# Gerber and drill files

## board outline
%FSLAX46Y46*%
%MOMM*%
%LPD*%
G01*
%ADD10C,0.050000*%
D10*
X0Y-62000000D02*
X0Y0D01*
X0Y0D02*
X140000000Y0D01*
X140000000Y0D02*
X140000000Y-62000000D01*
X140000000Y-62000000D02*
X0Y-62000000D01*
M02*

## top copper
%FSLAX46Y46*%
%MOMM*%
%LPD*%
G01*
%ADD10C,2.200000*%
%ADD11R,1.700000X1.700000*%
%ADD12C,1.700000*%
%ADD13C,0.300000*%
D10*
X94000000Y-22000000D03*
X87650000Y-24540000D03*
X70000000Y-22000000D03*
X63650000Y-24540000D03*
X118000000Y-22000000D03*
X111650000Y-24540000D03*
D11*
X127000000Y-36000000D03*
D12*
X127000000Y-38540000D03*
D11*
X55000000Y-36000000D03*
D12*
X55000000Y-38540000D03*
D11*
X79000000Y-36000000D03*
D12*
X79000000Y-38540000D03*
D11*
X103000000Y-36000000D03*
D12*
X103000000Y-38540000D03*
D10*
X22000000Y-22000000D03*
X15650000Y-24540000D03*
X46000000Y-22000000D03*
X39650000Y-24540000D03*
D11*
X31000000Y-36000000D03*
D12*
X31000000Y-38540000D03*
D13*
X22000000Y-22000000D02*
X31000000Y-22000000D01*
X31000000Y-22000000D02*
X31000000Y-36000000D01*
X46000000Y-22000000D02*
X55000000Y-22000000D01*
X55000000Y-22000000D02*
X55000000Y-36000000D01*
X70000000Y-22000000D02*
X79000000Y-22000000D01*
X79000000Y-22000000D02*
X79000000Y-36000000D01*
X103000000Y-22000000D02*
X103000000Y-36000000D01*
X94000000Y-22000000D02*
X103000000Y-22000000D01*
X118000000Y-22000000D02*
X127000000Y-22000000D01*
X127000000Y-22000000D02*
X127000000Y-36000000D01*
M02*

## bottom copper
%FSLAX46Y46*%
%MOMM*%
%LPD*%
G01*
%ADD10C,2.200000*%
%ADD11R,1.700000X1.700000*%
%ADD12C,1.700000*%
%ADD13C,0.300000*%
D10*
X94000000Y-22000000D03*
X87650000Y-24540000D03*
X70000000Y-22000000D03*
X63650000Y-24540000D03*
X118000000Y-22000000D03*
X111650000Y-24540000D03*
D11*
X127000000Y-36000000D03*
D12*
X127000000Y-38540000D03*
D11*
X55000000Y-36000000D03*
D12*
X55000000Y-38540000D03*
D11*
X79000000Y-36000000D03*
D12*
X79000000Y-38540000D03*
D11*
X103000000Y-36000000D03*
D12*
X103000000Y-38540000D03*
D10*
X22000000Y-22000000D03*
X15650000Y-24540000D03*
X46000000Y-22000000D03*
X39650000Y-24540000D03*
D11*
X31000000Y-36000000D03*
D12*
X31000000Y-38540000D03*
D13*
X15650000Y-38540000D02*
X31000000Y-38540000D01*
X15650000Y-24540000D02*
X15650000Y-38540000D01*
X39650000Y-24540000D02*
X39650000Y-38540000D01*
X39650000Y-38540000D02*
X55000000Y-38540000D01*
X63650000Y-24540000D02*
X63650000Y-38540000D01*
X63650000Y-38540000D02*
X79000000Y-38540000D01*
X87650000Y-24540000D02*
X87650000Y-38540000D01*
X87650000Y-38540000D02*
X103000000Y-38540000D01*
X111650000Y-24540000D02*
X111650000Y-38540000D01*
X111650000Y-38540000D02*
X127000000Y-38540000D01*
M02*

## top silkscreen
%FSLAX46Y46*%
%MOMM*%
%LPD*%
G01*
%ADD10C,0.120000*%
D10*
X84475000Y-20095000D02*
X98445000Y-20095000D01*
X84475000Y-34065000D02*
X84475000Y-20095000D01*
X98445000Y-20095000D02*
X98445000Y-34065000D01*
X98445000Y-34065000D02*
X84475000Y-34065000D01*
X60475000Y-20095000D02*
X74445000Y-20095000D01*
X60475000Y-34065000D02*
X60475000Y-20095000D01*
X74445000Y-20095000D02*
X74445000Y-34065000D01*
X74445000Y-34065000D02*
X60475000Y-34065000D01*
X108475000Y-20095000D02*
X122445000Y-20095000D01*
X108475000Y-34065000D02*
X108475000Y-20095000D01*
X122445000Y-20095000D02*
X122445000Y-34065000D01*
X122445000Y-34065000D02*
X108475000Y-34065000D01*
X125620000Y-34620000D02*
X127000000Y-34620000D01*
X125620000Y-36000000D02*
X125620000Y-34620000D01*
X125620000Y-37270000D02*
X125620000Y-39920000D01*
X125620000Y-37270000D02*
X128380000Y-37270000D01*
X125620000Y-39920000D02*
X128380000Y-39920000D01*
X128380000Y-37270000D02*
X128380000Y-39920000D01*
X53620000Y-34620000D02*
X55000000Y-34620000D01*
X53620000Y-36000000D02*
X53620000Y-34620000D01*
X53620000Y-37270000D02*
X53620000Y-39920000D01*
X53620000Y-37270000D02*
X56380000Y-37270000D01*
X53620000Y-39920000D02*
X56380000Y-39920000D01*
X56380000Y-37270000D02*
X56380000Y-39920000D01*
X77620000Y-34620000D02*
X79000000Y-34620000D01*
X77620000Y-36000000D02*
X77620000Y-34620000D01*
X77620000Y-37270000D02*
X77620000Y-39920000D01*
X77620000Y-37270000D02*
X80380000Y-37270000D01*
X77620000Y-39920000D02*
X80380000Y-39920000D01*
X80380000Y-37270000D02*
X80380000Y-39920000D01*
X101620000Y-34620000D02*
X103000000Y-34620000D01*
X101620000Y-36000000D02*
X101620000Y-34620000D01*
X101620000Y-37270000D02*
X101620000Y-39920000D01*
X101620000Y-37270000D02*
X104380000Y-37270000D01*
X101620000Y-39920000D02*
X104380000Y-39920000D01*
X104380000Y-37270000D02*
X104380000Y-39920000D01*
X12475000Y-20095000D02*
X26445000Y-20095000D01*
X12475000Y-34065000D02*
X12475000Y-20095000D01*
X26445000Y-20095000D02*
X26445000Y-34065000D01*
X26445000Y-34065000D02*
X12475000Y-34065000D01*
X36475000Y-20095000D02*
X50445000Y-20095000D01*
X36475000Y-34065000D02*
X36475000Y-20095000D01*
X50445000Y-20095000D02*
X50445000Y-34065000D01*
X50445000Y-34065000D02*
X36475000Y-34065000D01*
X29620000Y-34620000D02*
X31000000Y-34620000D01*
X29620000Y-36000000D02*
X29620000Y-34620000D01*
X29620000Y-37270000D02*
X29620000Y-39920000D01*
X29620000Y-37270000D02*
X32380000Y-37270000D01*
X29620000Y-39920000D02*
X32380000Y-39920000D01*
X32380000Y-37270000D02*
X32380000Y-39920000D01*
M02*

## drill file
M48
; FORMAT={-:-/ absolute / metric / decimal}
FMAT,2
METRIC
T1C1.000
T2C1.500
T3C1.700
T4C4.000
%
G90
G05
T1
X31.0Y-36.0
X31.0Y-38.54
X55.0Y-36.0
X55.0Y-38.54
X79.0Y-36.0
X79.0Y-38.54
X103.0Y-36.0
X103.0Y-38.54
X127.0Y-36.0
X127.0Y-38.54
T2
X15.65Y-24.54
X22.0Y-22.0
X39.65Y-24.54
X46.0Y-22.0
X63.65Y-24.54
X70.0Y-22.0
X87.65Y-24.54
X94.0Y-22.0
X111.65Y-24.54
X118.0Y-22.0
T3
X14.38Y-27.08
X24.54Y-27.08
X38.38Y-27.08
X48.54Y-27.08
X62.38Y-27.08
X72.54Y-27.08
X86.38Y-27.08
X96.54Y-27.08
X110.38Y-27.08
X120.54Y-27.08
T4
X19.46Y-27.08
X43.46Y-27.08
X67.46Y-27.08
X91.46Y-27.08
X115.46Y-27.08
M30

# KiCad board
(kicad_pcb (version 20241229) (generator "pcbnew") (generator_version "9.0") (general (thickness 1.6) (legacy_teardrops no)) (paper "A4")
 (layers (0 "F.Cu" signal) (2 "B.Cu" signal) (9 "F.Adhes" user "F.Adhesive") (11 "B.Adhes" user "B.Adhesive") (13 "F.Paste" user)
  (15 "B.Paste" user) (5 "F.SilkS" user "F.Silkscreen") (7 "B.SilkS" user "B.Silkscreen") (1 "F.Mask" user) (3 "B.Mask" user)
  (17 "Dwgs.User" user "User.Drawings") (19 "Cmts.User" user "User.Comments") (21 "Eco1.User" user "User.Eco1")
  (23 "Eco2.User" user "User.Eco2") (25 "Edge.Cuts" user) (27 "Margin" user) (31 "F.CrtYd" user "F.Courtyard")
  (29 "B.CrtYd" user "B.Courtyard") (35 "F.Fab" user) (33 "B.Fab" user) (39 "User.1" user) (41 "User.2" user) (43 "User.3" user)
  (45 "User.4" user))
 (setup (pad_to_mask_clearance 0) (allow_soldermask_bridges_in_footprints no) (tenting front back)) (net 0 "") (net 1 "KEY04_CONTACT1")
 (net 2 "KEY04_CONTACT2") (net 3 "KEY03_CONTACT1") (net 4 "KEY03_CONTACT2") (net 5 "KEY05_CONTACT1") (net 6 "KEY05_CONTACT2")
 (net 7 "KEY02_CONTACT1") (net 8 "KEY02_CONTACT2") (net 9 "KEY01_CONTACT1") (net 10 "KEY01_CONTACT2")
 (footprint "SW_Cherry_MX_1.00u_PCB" (layer "F.Cu") (at 94 22)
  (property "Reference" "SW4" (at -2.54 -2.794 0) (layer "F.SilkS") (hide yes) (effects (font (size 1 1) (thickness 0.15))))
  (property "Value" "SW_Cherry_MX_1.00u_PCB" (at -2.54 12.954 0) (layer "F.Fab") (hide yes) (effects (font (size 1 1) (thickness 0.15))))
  (fp_line (start -9.525 -1.905) (end 4.445 -1.905) (stroke (width 0.12) (type solid)) (layer "F.SilkS"))
  (fp_line (start -9.525 12.065) (end -9.525 -1.905) (stroke (width 0.12) (type solid)) (layer "F.SilkS"))
  (fp_line (start 4.445 -1.905) (end 4.445 12.065) (stroke (width 0.12) (type solid)) (layer "F.SilkS"))
  (fp_line (start 4.445 12.065) (end -9.525 12.065) (stroke (width 0.12) (type solid)) (layer "F.SilkS"))
  (pad "" np_thru_hole circle (at -7.62 5.08) (size 1.7 1.7) (drill 1.7) (layers "*.Cu" "*.Mask"))
  (pad "" np_thru_hole circle (at -2.54 5.08) (size 4 4) (drill 4) (layers "*.Cu" "*.Mask"))
  (pad "" np_thru_hole circle (at 2.54 5.08) (size 1.7 1.7) (drill 1.7) (layers "*.Cu" "*.Mask"))
  (pad "1" thru_hole circle (at 0 0) (size 2.2 2.2) (drill 1.5) (layers "*.Cu" "*.Mask") (remove_unused_layers no) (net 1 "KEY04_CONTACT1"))
  (pad "2" thru_hole circle (at -6.35 2.54) (size 2.2 2.2) (drill 1.5) (layers "*.Cu" "*.Mask") (remove_unused_layers no)
   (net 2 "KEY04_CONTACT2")))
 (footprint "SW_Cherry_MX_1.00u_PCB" (layer "F.Cu") (at 70 22)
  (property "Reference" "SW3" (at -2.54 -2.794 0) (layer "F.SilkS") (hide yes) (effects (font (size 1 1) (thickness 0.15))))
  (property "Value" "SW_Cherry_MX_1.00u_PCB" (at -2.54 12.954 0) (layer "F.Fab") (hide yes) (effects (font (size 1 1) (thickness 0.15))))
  (fp_line (start -9.525 -1.905) (end 4.445 -1.905) (stroke (width 0.12) (type solid)) (layer "F.SilkS"))
  (fp_line (start -9.525 12.065) (end -9.525 -1.905) (stroke (width 0.12) (type solid)) (layer "F.SilkS"))
  (fp_line (start 4.445 -1.905) (end 4.445 12.065) (stroke (width 0.12) (type solid)) (layer "F.SilkS"))
  (fp_line (start 4.445 12.065) (end -9.525 12.065) (stroke (width 0.12) (type solid)) (layer "F.SilkS"))
  (pad "" np_thru_hole circle (at -7.62 5.08) (size 1.7 1.7) (drill 1.7) (layers "*.Cu" "*.Mask"))
  (pad "" np_thru_hole circle (at -2.54 5.08) (size 4 4) (drill 4) (layers "*.Cu" "*.Mask"))
  (pad "" np_thru_hole circle (at 2.54 5.08) (size 1.7 1.7) (drill 1.7) (layers "*.Cu" "*.Mask"))
  (pad "1" thru_hole circle (at 0 0) (size 2.2 2.2) (drill 1.5) (layers "*.Cu" "*.Mask") (remove_unused_layers no) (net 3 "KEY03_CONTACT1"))
  (pad "2" thru_hole circle (at -6.35 2.54) (size 2.2 2.2) (drill 1.5) (layers "*.Cu" "*.Mask") (remove_unused_layers no)
   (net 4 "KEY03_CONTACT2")))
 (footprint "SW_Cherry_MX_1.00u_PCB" (layer "F.Cu") (at 118 22)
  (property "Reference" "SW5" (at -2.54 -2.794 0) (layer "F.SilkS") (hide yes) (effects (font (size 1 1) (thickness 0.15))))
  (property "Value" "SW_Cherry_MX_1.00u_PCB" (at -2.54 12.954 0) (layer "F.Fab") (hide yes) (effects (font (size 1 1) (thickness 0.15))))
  (fp_line (start -9.525 -1.905) (end 4.445 -1.905) (stroke (width 0.12) (type solid)) (layer "F.SilkS"))
  (fp_line (start -9.525 12.065) (end -9.525 -1.905) (stroke (width 0.12) (type solid)) (layer "F.SilkS"))
  (fp_line (start 4.445 -1.905) (end 4.445 12.065) (stroke (width 0.12) (type solid)) (layer "F.SilkS"))
  (fp_line (start 4.445 12.065) (end -9.525 12.065) (stroke (width 0.12) (type solid)) (layer "F.SilkS"))
  (pad "" np_thru_hole circle (at -7.62 5.08) (size 1.7 1.7) (drill 1.7) (layers "*.Cu" "*.Mask"))
  (pad "" np_thru_hole circle (at -2.54 5.08) (size 4 4) (drill 4) (layers "*.Cu" "*.Mask"))
  (pad "" np_thru_hole circle (at 2.54 5.08) (size 1.7 1.7) (drill 1.7) (layers "*.Cu" "*.Mask"))
  (pad "1" thru_hole circle (at 0 0) (size 2.2 2.2) (drill 1.5) (layers "*.Cu" "*.Mask") (remove_unused_layers no) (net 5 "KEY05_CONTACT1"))
  (pad "2" thru_hole circle (at -6.35 2.54) (size 2.2 2.2) (drill 1.5) (layers "*.Cu" "*.Mask") (remove_unused_layers no)
   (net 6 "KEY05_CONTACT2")))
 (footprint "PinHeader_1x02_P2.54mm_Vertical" (layer "F.Cu") (at 127 36)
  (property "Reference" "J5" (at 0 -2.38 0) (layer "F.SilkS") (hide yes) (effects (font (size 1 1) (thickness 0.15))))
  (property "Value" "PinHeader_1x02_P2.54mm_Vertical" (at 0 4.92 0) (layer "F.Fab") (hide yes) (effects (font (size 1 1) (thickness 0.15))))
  (fp_line (start -1.38 -1.38) (end 0 -1.38) (stroke (width 0.12) (type solid)) (layer "F.SilkS"))
  (fp_line (start -1.38 0) (end -1.38 -1.38) (stroke (width 0.12) (type solid)) (layer "F.SilkS"))
  (fp_line (start -1.38 1.27) (end -1.38 3.92) (stroke (width 0.12) (type solid)) (layer "F.SilkS"))
  (fp_line (start -1.38 1.27) (end 1.38 1.27) (stroke (width 0.12) (type solid)) (layer "F.SilkS"))
  (fp_line (start -1.38 3.92) (end 1.38 3.92) (stroke (width 0.12) (type solid)) (layer "F.SilkS"))
  (fp_line (start 1.38 1.27) (end 1.38 3.92) (stroke (width 0.12) (type solid)) (layer "F.SilkS"))
  (pad "1" thru_hole rect (at 0 0) (size 1.7 1.7) (drill 1) (layers "*.Cu" "*.Mask") (remove_unused_layers no) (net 5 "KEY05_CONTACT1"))
  (pad "2" thru_hole circle (at 0 2.54) (size 1.7 1.7) (drill 1) (layers "*.Cu" "*.Mask") (remove_unused_layers no) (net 6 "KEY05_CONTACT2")))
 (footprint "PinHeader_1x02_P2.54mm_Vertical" (layer "F.Cu") (at 55 36)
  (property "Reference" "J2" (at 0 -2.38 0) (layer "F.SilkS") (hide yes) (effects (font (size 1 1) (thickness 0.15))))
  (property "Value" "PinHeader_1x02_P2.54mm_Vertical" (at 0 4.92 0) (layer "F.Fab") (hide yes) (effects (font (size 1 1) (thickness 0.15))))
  (fp_line (start -1.38 -1.38) (end 0 -1.38) (stroke (width 0.12) (type solid)) (layer "F.SilkS"))
  (fp_line (start -1.38 0) (end -1.38 -1.38) (stroke (width 0.12) (type solid)) (layer "F.SilkS"))
  (fp_line (start -1.38 1.27) (end -1.38 3.92) (stroke (width 0.12) (type solid)) (layer "F.SilkS"))
  (fp_line (start -1.38 1.27) (end 1.38 1.27) (stroke (width 0.12) (type solid)) (layer "F.SilkS"))
  (fp_line (start -1.38 3.92) (end 1.38 3.92) (stroke (width 0.12) (type solid)) (layer "F.SilkS"))
  (fp_line (start 1.38 1.27) (end 1.38 3.92) (stroke (width 0.12) (type solid)) (layer "F.SilkS"))
  (pad "1" thru_hole rect (at 0 0) (size 1.7 1.7) (drill 1) (layers "*.Cu" "*.Mask") (remove_unused_layers no) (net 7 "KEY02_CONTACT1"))
  (pad "2" thru_hole circle (at 0 2.54) (size 1.7 1.7) (drill 1) (layers "*.Cu" "*.Mask") (remove_unused_layers no) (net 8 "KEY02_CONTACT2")))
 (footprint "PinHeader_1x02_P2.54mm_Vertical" (layer "F.Cu") (at 79 36)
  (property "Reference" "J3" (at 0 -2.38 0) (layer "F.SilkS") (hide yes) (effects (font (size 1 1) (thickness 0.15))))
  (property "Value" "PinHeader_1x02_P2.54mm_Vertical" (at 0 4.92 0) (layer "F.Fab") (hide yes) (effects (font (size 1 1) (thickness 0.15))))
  (fp_line (start -1.38 -1.38) (end 0 -1.38) (stroke (width 0.12) (type solid)) (layer "F.SilkS"))
  (fp_line (start -1.38 0) (end -1.38 -1.38) (stroke (width 0.12) (type solid)) (layer "F.SilkS"))
  (fp_line (start -1.38 1.27) (end -1.38 3.92) (stroke (width 0.12) (type solid)) (layer "F.SilkS"))
  (fp_line (start -1.38 1.27) (end 1.38 1.27) (stroke (width 0.12) (type solid)) (layer "F.SilkS"))
  (fp_line (start -1.38 3.92) (end 1.38 3.92) (stroke (width 0.12) (type solid)) (layer "F.SilkS"))
  (fp_line (start 1.38 1.27) (end 1.38 3.92) (stroke (width 0.12) (type solid)) (layer "F.SilkS"))
  (pad "1" thru_hole rect (at 0 0) (size 1.7 1.7) (drill 1) (layers "*.Cu" "*.Mask") (remove_unused_layers no) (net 3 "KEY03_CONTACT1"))
  (pad "2" thru_hole circle (at 0 2.54) (size 1.7 1.7) (drill 1) (layers "*.Cu" "*.Mask") (remove_unused_layers no) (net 4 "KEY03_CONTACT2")))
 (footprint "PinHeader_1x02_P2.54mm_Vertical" (layer "F.Cu") (at 103 36)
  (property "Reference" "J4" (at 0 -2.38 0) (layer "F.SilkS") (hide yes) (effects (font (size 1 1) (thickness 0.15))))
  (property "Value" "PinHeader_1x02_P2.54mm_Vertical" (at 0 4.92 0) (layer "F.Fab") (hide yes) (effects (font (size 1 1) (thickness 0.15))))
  (fp_line (start -1.38 -1.38) (end 0 -1.38) (stroke (width 0.12) (type solid)) (layer "F.SilkS"))
  (fp_line (start -1.38 0) (end -1.38 -1.38) (stroke (width 0.12) (type solid)) (layer "F.SilkS"))
  (fp_line (start -1.38 1.27) (end -1.38 3.92) (stroke (width 0.12) (type solid)) (layer "F.SilkS"))
  (fp_line (start -1.38 1.27) (end 1.38 1.27) (stroke (width 0.12) (type solid)) (layer "F.SilkS"))
  (fp_line (start -1.38 3.92) (end 1.38 3.92) (stroke (width 0.12) (type solid)) (layer "F.SilkS"))
  (fp_line (start 1.38 1.27) (end 1.38 3.92) (stroke (width 0.12) (type solid)) (layer "F.SilkS"))
  (pad "1" thru_hole rect (at 0 0) (size 1.7 1.7) (drill 1) (layers "*.Cu" "*.Mask") (remove_unused_layers no) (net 1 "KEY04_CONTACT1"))
  (pad "2" thru_hole circle (at 0 2.54) (size 1.7 1.7) (drill 1) (layers "*.Cu" "*.Mask") (remove_unused_layers no) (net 2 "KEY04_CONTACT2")))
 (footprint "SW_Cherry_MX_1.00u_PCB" (layer "F.Cu") (at 22 22)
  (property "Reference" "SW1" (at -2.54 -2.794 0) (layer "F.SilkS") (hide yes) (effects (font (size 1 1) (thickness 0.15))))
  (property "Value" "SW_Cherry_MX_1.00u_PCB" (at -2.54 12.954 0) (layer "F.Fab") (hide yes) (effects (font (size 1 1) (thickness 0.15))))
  (fp_line (start -9.525 -1.905) (end 4.445 -1.905) (stroke (width 0.12) (type solid)) (layer "F.SilkS"))
  (fp_line (start -9.525 12.065) (end -9.525 -1.905) (stroke (width 0.12) (type solid)) (layer "F.SilkS"))
  (fp_line (start 4.445 -1.905) (end 4.445 12.065) (stroke (width 0.12) (type solid)) (layer "F.SilkS"))
  (fp_line (start 4.445 12.065) (end -9.525 12.065) (stroke (width 0.12) (type solid)) (layer "F.SilkS"))
  (pad "" np_thru_hole circle (at -7.62 5.08) (size 1.7 1.7) (drill 1.7) (layers "*.Cu" "*.Mask"))
  (pad "" np_thru_hole circle (at -2.54 5.08) (size 4 4) (drill 4) (layers "*.Cu" "*.Mask"))
  (pad "" np_thru_hole circle (at 2.54 5.08) (size 1.7 1.7) (drill 1.7) (layers "*.Cu" "*.Mask"))
  (pad "1" thru_hole circle (at 0 0) (size 2.2 2.2) (drill 1.5) (layers "*.Cu" "*.Mask") (remove_unused_layers no) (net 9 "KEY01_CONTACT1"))
  (pad "2" thru_hole circle (at -6.35 2.54) (size 2.2 2.2) (drill 1.5) (layers "*.Cu" "*.Mask") (remove_unused_layers no)
   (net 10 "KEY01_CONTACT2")))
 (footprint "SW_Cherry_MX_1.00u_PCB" (layer "F.Cu") (at 46 22)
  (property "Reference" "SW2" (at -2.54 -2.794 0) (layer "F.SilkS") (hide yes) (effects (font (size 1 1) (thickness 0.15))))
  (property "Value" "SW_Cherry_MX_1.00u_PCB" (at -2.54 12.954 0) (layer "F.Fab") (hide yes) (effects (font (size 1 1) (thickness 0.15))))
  (fp_line (start -9.525 -1.905) (end 4.445 -1.905) (stroke (width 0.12) (type solid)) (layer "F.SilkS"))
  (fp_line (start -9.525 12.065) (end -9.525 -1.905) (stroke (width 0.12) (type solid)) (layer "F.SilkS"))
  (fp_line (start 4.445 -1.905) (end 4.445 12.065) (stroke (width 0.12) (type solid)) (layer "F.SilkS"))
  (fp_line (start 4.445 12.065) (end -9.525 12.065) (stroke (width 0.12) (type solid)) (layer "F.SilkS"))
  (pad "" np_thru_hole circle (at -7.62 5.08) (size 1.7 1.7) (drill 1.7) (layers "*.Cu" "*.Mask"))
  (pad "" np_thru_hole circle (at -2.54 5.08) (size 4 4) (drill 4) (layers "*.Cu" "*.Mask"))
  (pad "" np_thru_hole circle (at 2.54 5.08) (size 1.7 1.7) (drill 1.7) (layers "*.Cu" "*.Mask"))
  (pad "1" thru_hole circle (at 0 0) (size 2.2 2.2) (drill 1.5) (layers "*.Cu" "*.Mask") (remove_unused_layers no) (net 7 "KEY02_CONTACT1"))
  (pad "2" thru_hole circle (at -6.35 2.54) (size 2.2 2.2) (drill 1.5) (layers "*.Cu" "*.Mask") (remove_unused_layers no)
   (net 8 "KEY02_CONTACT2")))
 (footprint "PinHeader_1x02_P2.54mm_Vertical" (layer "F.Cu") (at 31 36)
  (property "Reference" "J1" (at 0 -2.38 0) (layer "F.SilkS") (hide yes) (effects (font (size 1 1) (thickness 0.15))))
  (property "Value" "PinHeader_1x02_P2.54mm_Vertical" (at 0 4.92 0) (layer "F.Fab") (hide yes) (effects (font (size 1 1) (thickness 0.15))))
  (fp_line (start -1.38 -1.38) (end 0 -1.38) (stroke (width 0.12) (type solid)) (layer "F.SilkS"))
  (fp_line (start -1.38 0) (end -1.38 -1.38) (stroke (width 0.12) (type solid)) (layer "F.SilkS"))
  (fp_line (start -1.38 1.27) (end -1.38 3.92) (stroke (width 0.12) (type solid)) (layer "F.SilkS"))
  (fp_line (start -1.38 1.27) (end 1.38 1.27) (stroke (width 0.12) (type solid)) (layer "F.SilkS"))
  (fp_line (start -1.38 3.92) (end 1.38 3.92) (stroke (width 0.12) (type solid)) (layer "F.SilkS"))
  (fp_line (start 1.38 1.27) (end 1.38 3.92) (stroke (width 0.12) (type solid)) (layer "F.SilkS"))
  (pad "1" thru_hole rect (at 0 0) (size 1.7 1.7) (drill 1) (layers "*.Cu" "*.Mask") (remove_unused_layers no) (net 9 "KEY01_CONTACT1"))
  (pad "2" thru_hole circle (at 0 2.54) (size 1.7 1.7) (drill 1) (layers "*.Cu" "*.Mask") (remove_unused_layers no)
   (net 10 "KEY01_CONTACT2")))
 (gr_line (start 0 62) (end 0 0) (stroke (width 0.05) (type default)) (layer "Edge.Cuts"))
 (gr_line (start 0 0) (end 140 0) (stroke (width 0.05) (type default)) (layer "Edge.Cuts"))
 (gr_line (start 140 0) (end 140 62) (stroke (width 0.05) (type default)) (layer "Edge.Cuts"))
 (gr_line (start 140 62) (end 0 62) (stroke (width 0.05) (type default)) (layer "Edge.Cuts"))
 (segment (start 22 22) (end 31 22) (width 0.3) (layer "F.Cu") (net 9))
 (segment (start 31 22) (end 31 36) (width 0.3) (layer "F.Cu") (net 9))
 (segment (start 15.65 38.54) (end 31 38.54) (width 0.3) (layer "B.Cu") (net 10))
 (segment (start 15.65 24.54) (end 15.65 38.54) (width 0.3) (layer "B.Cu") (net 10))
 (segment (start 46 22) (end 55 22) (width 0.3) (layer "F.Cu") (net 7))
 (segment (start 55 22) (end 55 36) (width 0.3) (layer "F.Cu") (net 7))
 (segment (start 39.65 24.54) (end 39.65 38.54) (width 0.3) (layer "B.Cu") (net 8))
 (segment (start 39.65 38.54) (end 55 38.54) (width 0.3) (layer "B.Cu") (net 8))
 (segment (start 70 22) (end 79 22) (width 0.3) (layer "F.Cu") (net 3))
 (segment (start 79 22) (end 79 36) (width 0.3) (layer "F.Cu") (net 3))
 (segment (start 63.65 24.54) (end 63.65 38.54) (width 0.3) (layer "B.Cu") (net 4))
 (segment (start 63.65 38.54) (end 79 38.54) (width 0.3) (layer "B.Cu") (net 4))
 (segment (start 103 22) (end 103 36) (width 0.3) (layer "F.Cu") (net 1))
 (segment (start 94 22) (end 103 22) (width 0.3) (layer "F.Cu") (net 1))
 (segment (start 87.65 24.54) (end 87.65 38.54) (width 0.3) (layer "B.Cu") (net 2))
 (segment (start 87.65 38.54) (end 103 38.54) (width 0.3) (layer "B.Cu") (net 2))
 (segment (start 118 22) (end 127 22) (width 0.3) (layer "F.Cu") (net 5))
 (segment (start 127 22) (end 127 36) (width 0.3) (layer "F.Cu") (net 5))
 (segment (start 111.65 24.54) (end 111.65 38.54) (width 0.3) (layer "B.Cu") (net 6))
 (segment (start 111.65 38.54) (end 127 38.54) (width 0.3) (layer "B.Cu") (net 6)))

